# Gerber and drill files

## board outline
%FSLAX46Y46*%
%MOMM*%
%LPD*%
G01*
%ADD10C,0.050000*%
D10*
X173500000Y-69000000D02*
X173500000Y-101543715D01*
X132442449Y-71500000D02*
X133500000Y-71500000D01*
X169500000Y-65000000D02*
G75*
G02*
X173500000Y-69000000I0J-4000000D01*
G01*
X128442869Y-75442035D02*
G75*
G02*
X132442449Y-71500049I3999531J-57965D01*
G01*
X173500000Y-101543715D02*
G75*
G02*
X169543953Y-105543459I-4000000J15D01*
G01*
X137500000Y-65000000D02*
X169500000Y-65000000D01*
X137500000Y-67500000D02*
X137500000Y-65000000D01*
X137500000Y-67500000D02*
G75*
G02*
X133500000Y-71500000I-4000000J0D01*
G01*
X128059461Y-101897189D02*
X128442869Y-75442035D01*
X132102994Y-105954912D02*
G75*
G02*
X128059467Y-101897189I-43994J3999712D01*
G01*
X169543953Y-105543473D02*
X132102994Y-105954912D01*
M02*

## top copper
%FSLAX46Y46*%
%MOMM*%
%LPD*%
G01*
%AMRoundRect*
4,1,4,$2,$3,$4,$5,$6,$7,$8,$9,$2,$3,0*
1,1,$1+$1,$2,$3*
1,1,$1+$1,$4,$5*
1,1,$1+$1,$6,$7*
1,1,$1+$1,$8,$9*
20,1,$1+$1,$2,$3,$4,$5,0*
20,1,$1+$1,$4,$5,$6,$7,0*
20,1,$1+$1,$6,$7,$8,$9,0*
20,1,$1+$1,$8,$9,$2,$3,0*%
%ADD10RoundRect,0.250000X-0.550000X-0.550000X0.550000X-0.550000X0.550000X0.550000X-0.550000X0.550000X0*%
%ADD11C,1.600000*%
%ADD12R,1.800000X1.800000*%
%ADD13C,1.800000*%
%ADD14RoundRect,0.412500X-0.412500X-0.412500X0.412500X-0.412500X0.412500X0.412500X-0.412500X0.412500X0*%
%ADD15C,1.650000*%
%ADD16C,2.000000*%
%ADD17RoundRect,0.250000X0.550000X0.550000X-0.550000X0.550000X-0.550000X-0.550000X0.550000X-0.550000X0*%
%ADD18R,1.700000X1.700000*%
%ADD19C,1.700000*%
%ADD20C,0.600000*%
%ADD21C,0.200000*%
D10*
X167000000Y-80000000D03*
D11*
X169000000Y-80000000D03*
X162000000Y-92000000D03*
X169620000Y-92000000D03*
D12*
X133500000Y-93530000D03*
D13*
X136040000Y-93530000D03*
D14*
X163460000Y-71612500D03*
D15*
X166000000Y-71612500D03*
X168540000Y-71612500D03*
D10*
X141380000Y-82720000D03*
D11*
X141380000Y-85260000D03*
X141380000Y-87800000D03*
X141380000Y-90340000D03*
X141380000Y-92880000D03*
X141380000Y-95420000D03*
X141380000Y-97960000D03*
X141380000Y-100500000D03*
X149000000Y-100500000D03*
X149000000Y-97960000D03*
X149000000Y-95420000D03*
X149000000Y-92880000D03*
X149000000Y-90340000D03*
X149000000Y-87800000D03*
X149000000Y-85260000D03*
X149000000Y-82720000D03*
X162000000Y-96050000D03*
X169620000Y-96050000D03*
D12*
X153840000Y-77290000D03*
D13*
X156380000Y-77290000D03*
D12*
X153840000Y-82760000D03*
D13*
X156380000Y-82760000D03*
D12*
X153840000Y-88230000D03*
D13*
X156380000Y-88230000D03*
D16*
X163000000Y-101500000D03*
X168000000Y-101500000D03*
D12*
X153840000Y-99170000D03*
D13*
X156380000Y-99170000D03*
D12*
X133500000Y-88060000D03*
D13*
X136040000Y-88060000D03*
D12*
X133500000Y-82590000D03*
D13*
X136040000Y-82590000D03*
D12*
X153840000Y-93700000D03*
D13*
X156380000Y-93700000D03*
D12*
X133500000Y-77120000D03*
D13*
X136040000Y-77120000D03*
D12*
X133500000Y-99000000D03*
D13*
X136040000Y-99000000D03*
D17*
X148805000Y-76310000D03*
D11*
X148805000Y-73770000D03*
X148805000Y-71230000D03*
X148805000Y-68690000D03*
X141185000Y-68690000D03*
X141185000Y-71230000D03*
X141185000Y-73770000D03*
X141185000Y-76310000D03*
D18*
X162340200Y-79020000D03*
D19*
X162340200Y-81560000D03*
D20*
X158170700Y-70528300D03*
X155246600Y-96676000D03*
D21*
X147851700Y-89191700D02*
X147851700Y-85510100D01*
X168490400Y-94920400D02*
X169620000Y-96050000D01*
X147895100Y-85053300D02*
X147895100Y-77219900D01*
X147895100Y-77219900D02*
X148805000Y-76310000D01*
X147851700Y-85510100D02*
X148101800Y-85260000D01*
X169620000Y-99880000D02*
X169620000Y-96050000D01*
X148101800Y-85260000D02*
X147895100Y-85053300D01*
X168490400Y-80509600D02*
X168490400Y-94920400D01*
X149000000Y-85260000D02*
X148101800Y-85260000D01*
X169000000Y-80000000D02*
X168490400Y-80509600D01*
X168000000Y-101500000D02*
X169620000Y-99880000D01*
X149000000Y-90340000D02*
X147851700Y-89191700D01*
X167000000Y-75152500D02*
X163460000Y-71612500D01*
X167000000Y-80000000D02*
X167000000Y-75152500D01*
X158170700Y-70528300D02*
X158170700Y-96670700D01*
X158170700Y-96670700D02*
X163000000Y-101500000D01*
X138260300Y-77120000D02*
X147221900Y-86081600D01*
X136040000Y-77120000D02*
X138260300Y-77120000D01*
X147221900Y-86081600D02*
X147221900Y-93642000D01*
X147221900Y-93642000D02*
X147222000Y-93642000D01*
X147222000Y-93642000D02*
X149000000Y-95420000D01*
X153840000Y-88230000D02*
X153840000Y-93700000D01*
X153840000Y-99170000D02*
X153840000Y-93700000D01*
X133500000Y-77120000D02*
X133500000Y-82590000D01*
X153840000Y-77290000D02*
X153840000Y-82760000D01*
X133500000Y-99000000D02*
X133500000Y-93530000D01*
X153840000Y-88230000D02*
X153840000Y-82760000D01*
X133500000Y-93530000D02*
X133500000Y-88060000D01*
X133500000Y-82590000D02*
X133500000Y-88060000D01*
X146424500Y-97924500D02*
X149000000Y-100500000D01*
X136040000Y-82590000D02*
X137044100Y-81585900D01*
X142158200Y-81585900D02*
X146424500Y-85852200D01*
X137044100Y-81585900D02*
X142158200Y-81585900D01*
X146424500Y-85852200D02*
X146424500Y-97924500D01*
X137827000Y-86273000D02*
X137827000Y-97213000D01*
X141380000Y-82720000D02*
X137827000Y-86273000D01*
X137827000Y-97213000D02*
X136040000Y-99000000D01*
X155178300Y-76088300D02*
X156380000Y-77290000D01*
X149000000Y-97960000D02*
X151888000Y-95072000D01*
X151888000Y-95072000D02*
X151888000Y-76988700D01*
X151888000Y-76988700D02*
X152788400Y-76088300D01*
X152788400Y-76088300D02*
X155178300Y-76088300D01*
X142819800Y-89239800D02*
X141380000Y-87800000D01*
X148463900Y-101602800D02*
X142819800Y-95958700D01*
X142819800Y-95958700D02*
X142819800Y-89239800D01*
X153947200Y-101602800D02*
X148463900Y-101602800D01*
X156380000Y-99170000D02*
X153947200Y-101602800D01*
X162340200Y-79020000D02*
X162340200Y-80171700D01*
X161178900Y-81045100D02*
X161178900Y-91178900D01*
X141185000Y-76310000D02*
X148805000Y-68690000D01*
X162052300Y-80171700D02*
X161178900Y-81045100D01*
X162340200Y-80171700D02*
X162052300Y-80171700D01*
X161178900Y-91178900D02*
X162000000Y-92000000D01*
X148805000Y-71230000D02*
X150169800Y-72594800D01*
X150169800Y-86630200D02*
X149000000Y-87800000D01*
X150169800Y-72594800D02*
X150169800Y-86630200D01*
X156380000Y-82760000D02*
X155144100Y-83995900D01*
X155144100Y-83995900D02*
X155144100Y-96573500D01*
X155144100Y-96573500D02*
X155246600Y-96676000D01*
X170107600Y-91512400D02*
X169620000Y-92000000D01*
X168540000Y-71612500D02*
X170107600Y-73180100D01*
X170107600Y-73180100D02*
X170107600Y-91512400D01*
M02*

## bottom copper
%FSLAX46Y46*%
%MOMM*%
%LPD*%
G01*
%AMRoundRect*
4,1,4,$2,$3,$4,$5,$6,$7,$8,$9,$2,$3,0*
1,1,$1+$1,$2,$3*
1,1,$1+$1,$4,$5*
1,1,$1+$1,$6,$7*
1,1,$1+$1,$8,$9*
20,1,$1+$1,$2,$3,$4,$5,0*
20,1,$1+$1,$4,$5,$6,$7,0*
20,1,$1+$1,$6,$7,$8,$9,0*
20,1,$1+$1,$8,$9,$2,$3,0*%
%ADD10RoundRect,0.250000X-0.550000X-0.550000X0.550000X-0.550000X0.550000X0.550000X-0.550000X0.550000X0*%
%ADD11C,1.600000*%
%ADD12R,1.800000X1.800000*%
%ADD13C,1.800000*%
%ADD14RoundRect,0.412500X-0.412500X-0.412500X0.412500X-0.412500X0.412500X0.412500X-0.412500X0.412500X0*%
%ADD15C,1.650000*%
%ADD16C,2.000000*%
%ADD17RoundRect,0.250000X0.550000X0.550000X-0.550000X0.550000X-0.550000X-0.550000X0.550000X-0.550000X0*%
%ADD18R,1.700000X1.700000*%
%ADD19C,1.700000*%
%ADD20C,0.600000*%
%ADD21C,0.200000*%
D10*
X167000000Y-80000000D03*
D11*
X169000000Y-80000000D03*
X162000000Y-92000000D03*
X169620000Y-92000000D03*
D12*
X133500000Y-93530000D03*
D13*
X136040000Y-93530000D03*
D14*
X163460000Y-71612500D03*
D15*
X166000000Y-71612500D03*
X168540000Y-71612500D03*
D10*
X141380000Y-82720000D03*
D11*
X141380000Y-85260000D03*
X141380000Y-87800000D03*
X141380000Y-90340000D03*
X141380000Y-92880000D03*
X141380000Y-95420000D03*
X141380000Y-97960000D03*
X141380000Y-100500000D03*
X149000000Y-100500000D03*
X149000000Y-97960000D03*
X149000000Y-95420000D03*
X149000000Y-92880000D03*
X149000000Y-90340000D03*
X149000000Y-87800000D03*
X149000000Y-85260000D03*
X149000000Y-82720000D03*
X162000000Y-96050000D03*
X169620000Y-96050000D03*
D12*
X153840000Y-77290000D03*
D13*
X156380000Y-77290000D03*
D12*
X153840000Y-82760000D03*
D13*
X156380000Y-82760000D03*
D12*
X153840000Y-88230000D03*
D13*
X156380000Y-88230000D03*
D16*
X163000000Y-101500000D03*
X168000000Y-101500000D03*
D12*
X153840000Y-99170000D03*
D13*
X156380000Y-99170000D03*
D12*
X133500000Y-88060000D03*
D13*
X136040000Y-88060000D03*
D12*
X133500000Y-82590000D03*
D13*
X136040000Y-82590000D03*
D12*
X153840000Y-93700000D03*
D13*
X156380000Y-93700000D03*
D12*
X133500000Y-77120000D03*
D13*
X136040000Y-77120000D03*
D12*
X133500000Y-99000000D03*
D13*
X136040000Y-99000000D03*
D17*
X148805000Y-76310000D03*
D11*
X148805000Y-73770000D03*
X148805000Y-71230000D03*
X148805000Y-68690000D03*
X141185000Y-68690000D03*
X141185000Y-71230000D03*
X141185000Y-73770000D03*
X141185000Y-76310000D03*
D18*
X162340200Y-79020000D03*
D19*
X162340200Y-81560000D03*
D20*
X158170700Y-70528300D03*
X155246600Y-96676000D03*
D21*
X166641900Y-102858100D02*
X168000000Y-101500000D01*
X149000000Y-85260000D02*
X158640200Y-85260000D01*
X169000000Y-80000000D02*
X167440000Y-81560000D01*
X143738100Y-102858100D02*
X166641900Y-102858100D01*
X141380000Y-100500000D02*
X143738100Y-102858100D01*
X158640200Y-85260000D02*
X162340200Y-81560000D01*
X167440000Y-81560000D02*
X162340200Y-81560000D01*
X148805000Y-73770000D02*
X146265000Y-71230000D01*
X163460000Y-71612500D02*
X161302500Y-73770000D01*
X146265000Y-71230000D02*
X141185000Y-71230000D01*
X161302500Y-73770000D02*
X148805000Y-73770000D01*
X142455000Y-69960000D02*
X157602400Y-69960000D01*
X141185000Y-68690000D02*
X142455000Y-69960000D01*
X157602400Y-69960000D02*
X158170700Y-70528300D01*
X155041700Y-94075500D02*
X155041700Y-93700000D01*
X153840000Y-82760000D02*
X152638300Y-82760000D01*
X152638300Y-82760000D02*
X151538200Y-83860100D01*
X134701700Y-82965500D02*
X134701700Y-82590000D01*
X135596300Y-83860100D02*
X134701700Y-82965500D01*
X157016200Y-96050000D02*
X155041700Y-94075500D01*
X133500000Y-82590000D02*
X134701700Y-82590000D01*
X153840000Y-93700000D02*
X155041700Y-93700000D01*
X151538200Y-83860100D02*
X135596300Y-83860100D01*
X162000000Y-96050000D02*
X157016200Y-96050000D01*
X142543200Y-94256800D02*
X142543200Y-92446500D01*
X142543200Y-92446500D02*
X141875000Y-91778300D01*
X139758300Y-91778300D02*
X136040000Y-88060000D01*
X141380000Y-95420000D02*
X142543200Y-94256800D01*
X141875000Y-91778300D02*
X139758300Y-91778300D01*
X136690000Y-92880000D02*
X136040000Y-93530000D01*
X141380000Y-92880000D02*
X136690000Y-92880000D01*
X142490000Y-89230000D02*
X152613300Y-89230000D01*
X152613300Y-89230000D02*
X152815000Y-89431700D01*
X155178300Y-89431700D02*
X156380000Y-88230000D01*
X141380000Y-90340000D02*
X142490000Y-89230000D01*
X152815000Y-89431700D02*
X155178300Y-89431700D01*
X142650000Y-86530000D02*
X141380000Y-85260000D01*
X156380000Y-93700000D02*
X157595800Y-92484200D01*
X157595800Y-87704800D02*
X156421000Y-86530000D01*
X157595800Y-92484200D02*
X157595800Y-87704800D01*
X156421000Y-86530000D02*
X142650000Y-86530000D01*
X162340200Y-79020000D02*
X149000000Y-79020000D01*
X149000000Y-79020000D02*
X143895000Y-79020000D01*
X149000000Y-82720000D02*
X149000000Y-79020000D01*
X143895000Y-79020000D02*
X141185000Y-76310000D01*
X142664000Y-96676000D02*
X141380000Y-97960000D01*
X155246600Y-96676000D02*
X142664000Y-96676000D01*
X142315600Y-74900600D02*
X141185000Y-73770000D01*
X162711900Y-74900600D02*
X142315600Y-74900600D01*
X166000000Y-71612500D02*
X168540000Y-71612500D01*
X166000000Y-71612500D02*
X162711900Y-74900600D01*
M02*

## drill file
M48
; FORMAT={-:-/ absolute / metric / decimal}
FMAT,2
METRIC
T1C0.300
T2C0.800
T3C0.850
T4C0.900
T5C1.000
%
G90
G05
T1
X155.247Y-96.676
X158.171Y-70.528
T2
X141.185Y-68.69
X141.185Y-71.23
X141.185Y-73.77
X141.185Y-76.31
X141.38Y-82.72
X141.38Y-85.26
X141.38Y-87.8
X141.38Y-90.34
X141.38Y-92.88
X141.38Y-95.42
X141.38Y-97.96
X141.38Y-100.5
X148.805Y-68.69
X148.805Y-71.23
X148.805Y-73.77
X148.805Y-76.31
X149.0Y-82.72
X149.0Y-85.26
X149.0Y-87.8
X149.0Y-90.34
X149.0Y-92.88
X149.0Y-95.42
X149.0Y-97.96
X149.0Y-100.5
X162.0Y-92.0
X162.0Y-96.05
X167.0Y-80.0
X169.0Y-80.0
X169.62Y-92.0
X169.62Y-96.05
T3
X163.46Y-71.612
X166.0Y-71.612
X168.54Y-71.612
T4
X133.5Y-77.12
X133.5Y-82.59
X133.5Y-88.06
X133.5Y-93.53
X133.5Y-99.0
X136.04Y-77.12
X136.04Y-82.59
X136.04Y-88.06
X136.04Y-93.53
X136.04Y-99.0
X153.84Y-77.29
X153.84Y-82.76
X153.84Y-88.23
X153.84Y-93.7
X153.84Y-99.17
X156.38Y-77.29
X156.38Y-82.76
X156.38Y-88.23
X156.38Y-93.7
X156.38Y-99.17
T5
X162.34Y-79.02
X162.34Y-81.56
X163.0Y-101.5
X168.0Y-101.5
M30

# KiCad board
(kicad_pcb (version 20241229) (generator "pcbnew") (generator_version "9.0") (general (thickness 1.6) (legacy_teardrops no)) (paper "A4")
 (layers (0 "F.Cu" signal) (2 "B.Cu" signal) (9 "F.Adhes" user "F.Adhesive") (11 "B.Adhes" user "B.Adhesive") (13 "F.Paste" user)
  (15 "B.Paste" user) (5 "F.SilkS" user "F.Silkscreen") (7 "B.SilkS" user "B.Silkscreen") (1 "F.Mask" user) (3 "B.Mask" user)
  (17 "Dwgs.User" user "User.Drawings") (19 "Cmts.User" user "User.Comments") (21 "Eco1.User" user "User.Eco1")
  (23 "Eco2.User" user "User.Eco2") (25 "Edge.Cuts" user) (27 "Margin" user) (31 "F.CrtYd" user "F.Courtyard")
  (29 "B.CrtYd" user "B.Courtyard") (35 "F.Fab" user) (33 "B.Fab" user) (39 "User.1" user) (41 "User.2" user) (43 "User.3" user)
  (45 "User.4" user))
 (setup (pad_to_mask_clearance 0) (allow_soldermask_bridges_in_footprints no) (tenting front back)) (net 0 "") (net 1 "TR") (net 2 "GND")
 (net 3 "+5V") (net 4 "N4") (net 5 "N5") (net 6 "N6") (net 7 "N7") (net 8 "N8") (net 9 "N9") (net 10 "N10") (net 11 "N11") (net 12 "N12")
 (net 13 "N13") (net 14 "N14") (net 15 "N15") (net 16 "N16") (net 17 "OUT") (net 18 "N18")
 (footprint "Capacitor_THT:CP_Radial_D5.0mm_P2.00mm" (layer "F.Cu") (at 167 80)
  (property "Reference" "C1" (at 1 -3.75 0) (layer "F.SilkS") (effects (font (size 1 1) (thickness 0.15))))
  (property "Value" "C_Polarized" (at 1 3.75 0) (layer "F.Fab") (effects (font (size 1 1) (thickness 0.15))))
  (pad "1" thru_hole roundrect (at 0 0) (size 1.6 1.6) (drill 0.8) (layers "*.Cu" "*.Mask") (remove_unused_layers no)
   (roundrect_rratio 0.15625) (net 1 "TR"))
  (pad "2" thru_hole circle (at 2 0) (size 1.6 1.6) (drill 0.8) (layers "*.Cu" "*.Mask") (remove_unused_layers no) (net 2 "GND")))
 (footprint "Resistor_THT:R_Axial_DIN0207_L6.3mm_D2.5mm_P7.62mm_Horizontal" (layer "F.Cu") (at 162 92)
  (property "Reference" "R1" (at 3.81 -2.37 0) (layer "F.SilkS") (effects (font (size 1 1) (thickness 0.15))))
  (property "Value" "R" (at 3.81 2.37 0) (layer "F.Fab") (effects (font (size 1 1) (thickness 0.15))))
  (pad "1" thru_hole circle (at 0 0) (size 1.6 1.6) (drill 0.8) (layers "*.Cu" "*.Mask") (remove_unused_layers no) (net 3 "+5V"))
  (pad "2" thru_hole circle (at 7.62 0) (size 1.6 1.6) (drill 0.8) (layers "*.Cu" "*.Mask") (remove_unused_layers no) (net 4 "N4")))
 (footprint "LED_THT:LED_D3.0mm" (layer "F.Cu") (at 133.5 93.53)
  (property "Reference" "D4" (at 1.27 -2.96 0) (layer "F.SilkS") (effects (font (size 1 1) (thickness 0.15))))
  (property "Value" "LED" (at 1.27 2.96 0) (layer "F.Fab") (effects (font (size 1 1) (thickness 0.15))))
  (pad "1" thru_hole rect (at 0 0) (size 1.8 1.8) (drill 0.9) (layers "*.Cu" "*.Mask") (remove_unused_layers no) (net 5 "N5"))
  (pad "2" thru_hole circle (at 2.54 0) (size 1.8 1.8) (drill 0.9) (layers "*.Cu" "*.Mask") (remove_unused_layers no) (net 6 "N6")))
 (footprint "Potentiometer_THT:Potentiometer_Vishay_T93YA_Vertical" (layer "F.Cu") (at 163.46 71.6125)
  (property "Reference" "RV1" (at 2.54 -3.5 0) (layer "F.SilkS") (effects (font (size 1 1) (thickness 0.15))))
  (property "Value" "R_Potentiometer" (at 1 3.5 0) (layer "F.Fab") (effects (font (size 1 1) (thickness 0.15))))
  (pad "1" thru_hole roundrect (at 0 0) (size 1.65 1.65) (drill 0.85) (layers "*.Cu" "*.Mask") (remove_unused_layers no)
   (roundrect_rratio 0.25) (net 1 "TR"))
  (pad "2" thru_hole circle (at 2.54 0) (size 1.65 1.65) (drill 0.85) (layers "*.Cu" "*.Mask") (remove_unused_layers no) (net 4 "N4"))
  (pad "3" thru_hole circle (at 5.08 0) (size 1.65 1.65) (drill 0.85) (layers "*.Cu" "*.Mask") (remove_unused_layers no) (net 4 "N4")))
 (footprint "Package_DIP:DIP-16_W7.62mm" (layer "F.Cu") (at 141.38 82.72)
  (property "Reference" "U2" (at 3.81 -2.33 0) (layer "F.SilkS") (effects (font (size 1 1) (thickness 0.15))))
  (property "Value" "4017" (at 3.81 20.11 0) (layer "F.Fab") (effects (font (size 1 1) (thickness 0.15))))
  (pad "1" thru_hole roundrect (at 0 0) (size 1.6 1.6) (drill 0.8) (layers "*.Cu" "*.Mask") (remove_unused_layers no)
   (roundrect_rratio 0.15625) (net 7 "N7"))
  (pad "2" thru_hole circle (at 0 2.54) (size 1.6 1.6) (drill 0.8) (layers "*.Cu" "*.Mask") (remove_unused_layers no) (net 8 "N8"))
  (pad "3" thru_hole circle (at 0 5.08) (size 1.6 1.6) (drill 0.8) (layers "*.Cu" "*.Mask") (remove_unused_layers no) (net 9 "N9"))
  (pad "4" thru_hole circle (at 0 7.62) (size 1.6 1.6) (drill 0.8) (layers "*.Cu" "*.Mask") (remove_unused_layers no) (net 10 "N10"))
  (pad "5" thru_hole circle (at 0 10.16) (size 1.6 1.6) (drill 0.8) (layers "*.Cu" "*.Mask") (remove_unused_layers no) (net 6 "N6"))
  (pad "6" thru_hole circle (at 0 12.7) (size 1.6 1.6) (drill 0.8) (layers "*.Cu" "*.Mask") (remove_unused_layers no) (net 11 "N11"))
  (pad "7" thru_hole circle (at 0 15.24) (size 1.6 1.6) (drill 0.8) (layers "*.Cu" "*.Mask") (remove_unused_layers no) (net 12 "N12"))
  (pad "8" thru_hole circle (at 0 17.78) (size 1.6 1.6) (drill 0.8) (layers "*.Cu" "*.Mask") (remove_unused_layers no) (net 2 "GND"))
  (pad "9" thru_hole circle (at 7.62 17.78) (size 1.6 1.6) (drill 0.8) (layers "*.Cu" "*.Mask") (remove_unused_layers no) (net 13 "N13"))
  (pad "10" thru_hole circle (at 7.62 15.24) (size 1.6 1.6) (drill 0.8) (layers "*.Cu" "*.Mask") (remove_unused_layers no) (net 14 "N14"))
  (pad "11" thru_hole circle (at 7.62 12.7) (size 1.6 1.6) (drill 0.8) (layers "*.Cu" "*.Mask") (remove_unused_layers no) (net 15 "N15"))
  (pad "12" thru_hole circle (at 7.62 10.16) (size 1.6 1.6) (drill 0.8) (layers "*.Cu" "*.Mask") (remove_unused_layers no) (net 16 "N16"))
  (pad "13" thru_hole circle (at 7.62 7.62) (size 1.6 1.6) (drill 0.8) (layers "*.Cu" "*.Mask") (remove_unused_layers no) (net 2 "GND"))
  (pad "14" thru_hole circle (at 7.62 5.08) (size 1.6 1.6) (drill 0.8) (layers "*.Cu" "*.Mask") (remove_unused_layers no) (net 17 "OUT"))
  (pad "15" thru_hole circle (at 7.62 2.54) (size 1.6 1.6) (drill 0.8) (layers "*.Cu" "*.Mask") (remove_unused_layers no) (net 2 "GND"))
  (pad "16" thru_hole circle (at 7.62 0) (size 1.6 1.6) (drill 0.8) (layers "*.Cu" "*.Mask") (remove_unused_layers no) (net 3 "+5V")))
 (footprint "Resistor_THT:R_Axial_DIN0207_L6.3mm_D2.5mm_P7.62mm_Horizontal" (layer "F.Cu") (at 162 96.05)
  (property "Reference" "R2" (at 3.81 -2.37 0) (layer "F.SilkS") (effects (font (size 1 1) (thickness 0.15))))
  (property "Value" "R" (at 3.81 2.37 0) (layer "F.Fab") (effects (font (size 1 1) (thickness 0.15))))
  (pad "1" thru_hole circle (at 0 0) (size 1.6 1.6) (drill 0.8) (layers "*.Cu" "*.Mask") (remove_unused_layers no) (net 5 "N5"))
  (pad "2" thru_hole circle (at 7.62 0) (size 1.6 1.6) (drill 0.8) (layers "*.Cu" "*.Mask") (remove_unused_layers no) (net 2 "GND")))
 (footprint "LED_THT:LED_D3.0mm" (layer "F.Cu") (at 153.84 77.29)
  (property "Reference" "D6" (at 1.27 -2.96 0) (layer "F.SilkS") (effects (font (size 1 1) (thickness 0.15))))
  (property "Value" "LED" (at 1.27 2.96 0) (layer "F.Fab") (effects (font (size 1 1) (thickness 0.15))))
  (pad "1" thru_hole rect (at 0 0) (size 1.8 1.8) (drill 0.9) (layers "*.Cu" "*.Mask") (remove_unused_layers no) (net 5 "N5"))
  (pad "2" thru_hole circle (at 2.54 0) (size 1.8 1.8) (drill 0.9) (layers "*.Cu" "*.Mask") (remove_unused_layers no) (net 14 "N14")))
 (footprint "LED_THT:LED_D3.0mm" (layer "F.Cu") (at 153.84 82.76)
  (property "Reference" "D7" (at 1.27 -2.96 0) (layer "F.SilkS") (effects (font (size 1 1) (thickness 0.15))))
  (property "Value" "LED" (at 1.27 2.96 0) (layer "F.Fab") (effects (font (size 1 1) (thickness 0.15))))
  (pad "1" thru_hole rect (at 0 0) (size 1.8 1.8) (drill 0.9) (layers "*.Cu" "*.Mask") (remove_unused_layers no) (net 5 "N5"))
  (pad "2" thru_hole circle (at 2.54 0) (size 1.8 1.8) (drill 0.9) (layers "*.Cu" "*.Mask") (remove_unused_layers no) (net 12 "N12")))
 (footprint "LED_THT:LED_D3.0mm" (layer "F.Cu") (at 153.84 88.23)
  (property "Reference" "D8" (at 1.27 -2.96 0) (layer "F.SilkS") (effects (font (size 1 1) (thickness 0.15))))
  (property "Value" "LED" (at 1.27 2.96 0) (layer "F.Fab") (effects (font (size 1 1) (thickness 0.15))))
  (pad "1" thru_hole rect (at 0 0) (size 1.8 1.8) (drill 0.9) (layers "*.Cu" "*.Mask") (remove_unused_layers no) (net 5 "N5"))
  (pad "2" thru_hole circle (at 2.54 0) (size 1.8 1.8) (drill 0.9) (layers "*.Cu" "*.Mask") (remove_unused_layers no) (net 10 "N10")))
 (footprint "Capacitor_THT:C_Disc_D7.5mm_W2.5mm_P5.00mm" (layer "F.Cu") (at 163 101.5)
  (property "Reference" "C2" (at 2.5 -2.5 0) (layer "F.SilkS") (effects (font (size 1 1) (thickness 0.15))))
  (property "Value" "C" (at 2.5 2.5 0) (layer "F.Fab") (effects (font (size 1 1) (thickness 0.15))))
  (pad "1" thru_hole circle (at 0 0) (size 2 2) (drill 1) (layers "*.Cu" "*.Mask") (remove_unused_layers no) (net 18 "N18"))
  (pad "2" thru_hole circle (at 5 0) (size 2 2) (drill 1) (layers "*.Cu" "*.Mask") (remove_unused_layers no) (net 2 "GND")))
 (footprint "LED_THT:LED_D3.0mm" (layer "F.Cu") (at 153.84 99.17)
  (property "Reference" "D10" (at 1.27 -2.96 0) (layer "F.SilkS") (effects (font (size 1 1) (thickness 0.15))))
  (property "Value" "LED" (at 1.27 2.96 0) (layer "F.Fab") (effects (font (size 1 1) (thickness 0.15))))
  (pad "1" thru_hole rect (at 0 0) (size 1.8 1.8) (drill 0.9) (layers "*.Cu" "*.Mask") (remove_unused_layers no) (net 5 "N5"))
  (pad "2" thru_hole circle (at 2.54 0) (size 1.8 1.8) (drill 0.9) (layers "*.Cu" "*.Mask") (remove_unused_layers no) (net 9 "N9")))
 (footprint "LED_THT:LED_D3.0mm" (layer "F.Cu") (at 133.5 88.06)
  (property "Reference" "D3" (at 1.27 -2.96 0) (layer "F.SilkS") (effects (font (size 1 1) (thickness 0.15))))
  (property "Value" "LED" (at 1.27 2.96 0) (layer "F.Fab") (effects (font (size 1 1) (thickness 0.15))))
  (pad "1" thru_hole rect (at 0 0) (size 1.8 1.8) (drill 0.9) (layers "*.Cu" "*.Mask") (remove_unused_layers no) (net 5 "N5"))
  (pad "2" thru_hole circle (at 2.54 0) (size 1.8 1.8) (drill 0.9) (layers "*.Cu" "*.Mask") (remove_unused_layers no) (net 11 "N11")))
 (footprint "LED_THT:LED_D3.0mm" (layer "F.Cu") (at 133.5 82.59)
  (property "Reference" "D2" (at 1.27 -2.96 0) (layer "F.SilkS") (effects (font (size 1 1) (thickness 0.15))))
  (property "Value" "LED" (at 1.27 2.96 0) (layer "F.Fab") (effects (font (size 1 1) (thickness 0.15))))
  (pad "1" thru_hole rect (at 0 0) (size 1.8 1.8) (drill 0.9) (layers "*.Cu" "*.Mask") (remove_unused_layers no) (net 5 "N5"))
  (pad "2" thru_hole circle (at 2.54 0) (size 1.8 1.8) (drill 0.9) (layers "*.Cu" "*.Mask") (remove_unused_layers no) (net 13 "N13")))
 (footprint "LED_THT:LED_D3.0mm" (layer "F.Cu") (at 153.84 93.7)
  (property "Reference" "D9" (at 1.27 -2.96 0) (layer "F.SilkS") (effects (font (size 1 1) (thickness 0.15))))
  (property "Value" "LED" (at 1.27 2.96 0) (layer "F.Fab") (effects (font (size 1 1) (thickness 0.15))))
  (pad "1" thru_hole rect (at 0 0) (size 1.8 1.8) (drill 0.9) (layers "*.Cu" "*.Mask") (remove_unused_layers no) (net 5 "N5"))
  (pad "2" thru_hole circle (at 2.54 0) (size 1.8 1.8) (drill 0.9) (layers "*.Cu" "*.Mask") (remove_unused_layers no) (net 8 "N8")))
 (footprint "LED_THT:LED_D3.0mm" (layer "F.Cu") (at 133.5 77.12)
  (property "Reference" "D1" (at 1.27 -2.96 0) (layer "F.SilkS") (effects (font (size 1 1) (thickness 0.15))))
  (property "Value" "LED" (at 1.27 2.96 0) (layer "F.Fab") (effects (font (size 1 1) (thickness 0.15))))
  (pad "1" thru_hole rect (at 0 0) (size 1.8 1.8) (drill 0.9) (layers "*.Cu" "*.Mask") (remove_unused_layers no) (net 5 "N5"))
  (pad "2" thru_hole circle (at 2.54 0) (size 1.8 1.8) (drill 0.9) (layers "*.Cu" "*.Mask") (remove_unused_layers no) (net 15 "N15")))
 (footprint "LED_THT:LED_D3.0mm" (layer "F.Cu") (at 133.5 99)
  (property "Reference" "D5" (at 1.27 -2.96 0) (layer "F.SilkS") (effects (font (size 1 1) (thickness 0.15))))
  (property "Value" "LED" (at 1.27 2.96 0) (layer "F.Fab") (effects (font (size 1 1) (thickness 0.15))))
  (pad "1" thru_hole rect (at 0 0) (size 1.8 1.8) (drill 0.9) (layers "*.Cu" "*.Mask") (remove_unused_layers no) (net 5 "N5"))
  (pad "2" thru_hole circle (at 2.54 0) (size 1.8 1.8) (drill 0.9) (layers "*.Cu" "*.Mask") (remove_unused_layers no) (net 7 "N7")))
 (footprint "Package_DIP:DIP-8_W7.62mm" (layer "F.Cu") (at 148.805 76.31 180)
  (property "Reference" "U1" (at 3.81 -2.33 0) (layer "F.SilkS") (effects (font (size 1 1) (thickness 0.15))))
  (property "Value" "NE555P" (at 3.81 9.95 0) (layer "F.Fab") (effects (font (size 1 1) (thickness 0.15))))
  (pad "1" thru_hole roundrect (at 0 0 180) (size 1.6 1.6) (drill 0.8) (layers "*.Cu" "*.Mask") (remove_unused_layers no)
   (roundrect_rratio 0.15625) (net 2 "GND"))
  (pad "2" thru_hole circle (at 0 2.54 180) (size 1.6 1.6) (drill 0.8) (layers "*.Cu" "*.Mask") (remove_unused_layers no) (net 1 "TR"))
  (pad "3" thru_hole circle (at 0 5.08 180) (size 1.6 1.6) (drill 0.8) (layers "*.Cu" "*.Mask") (remove_unused_layers no) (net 17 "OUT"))
  (pad "4" thru_hole circle (at 0 7.62 180) (size 1.6 1.6) (drill 0.8) (layers "*.Cu" "*.Mask") (remove_unused_layers no) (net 3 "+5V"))
  (pad "5" thru_hole circle (at 7.62 7.62 180) (size 1.6 1.6) (drill 0.8) (layers "*.Cu" "*.Mask") (remove_unused_layers no) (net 18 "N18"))
  (pad "6" thru_hole circle (at 7.62 5.08 180) (size 1.6 1.6) (drill 0.8) (layers "*.Cu" "*.Mask") (remove_unused_layers no) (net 1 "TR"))
  (pad "7" thru_hole circle (at 7.62 2.54 180) (size 1.6 1.6) (drill 0.8) (layers "*.Cu" "*.Mask") (remove_unused_layers no) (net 4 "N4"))
  (pad "8" thru_hole circle (at 7.62 0 180) (size 1.6 1.6) (drill 0.8) (layers "*.Cu" "*.Mask") (remove_unused_layers no) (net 3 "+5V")))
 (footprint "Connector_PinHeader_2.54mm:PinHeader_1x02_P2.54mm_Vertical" (layer "F.Cu") (at 162.3402 79.02)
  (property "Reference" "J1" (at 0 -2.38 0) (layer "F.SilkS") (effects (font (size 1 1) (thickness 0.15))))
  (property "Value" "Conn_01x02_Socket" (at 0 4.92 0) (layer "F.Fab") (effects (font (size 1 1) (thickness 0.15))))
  (pad "1" thru_hole rect (at 0 0) (size 1.7 1.7) (drill 1) (layers "*.Cu" "*.Mask") (remove_unused_layers no) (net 3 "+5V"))
  (pad "2" thru_hole circle (at 0 2.54) (size 1.7 1.7) (drill 1) (layers "*.Cu" "*.Mask") (remove_unused_layers no) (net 2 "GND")))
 (gr_line (start 173.5 69) (end 173.5 101.543715) (stroke (width 0.05) (type default)) (layer "Edge.Cuts"))
 (gr_line (start 132.442449 71.5) (end 133.5 71.5) (stroke (width 0.05) (type default)) (layer "Edge.Cuts"))
 (gr_arc (start 169.5 65) (mid 172.328427 66.171573) (end 173.5 69) (stroke (width 0.05) (type default)) (layer "Edge.Cuts"))
 (gr_arc (start 128.442869 75.442035) (mid 129.63459 72.651153) (end 132.442449 71.5) (stroke (width 0.05) (type default))
  (layer "Edge.Cuts"))
 (gr_arc (start 173.5 101.543715) (mid 172.343924 104.356559) (end 169.543953 105.543473) (stroke (width 0.05) (type default))
  (layer "Edge.Cuts"))
 (gr_line (start 137.5 65) (end 169.5 65) (stroke (width 0.05) (type default)) (layer "Edge.Cuts"))
 (gr_line (start 137.5 67.5) (end 137.5 65) (stroke (width 0.05) (type default)) (layer "Edge.Cuts"))
 (gr_arc (start 137.5 67.5) (mid 136.328427 70.328427) (end 133.5 71.5) (stroke (width 0.05) (type default)) (layer "Edge.Cuts"))
 (gr_line (start 128.059461 101.897189) (end 128.442869 75.442035) (stroke (width 0.05) (type default)) (layer "Edge.Cuts"))
 (gr_arc (start 132.102994 105.954912) (mid 129.225662 104.778623) (end 128.059461 101.897189) (stroke (width 0.05) (type default))
  (layer "Edge.Cuts"))
 (gr_line (start 169.543953 105.543473) (end 132.102994 105.954912) (stroke (width 0.05) (type default)) (layer "Edge.Cuts"))
 (segment (start 147.8517 89.1917) (end 147.8517 85.5101) (width 0.2) (layer "F.Cu") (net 2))
 (segment (start 168.4904 94.9204) (end 169.62 96.05) (width 0.2) (layer "F.Cu") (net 2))
 (segment (start 147.8951 85.0533) (end 147.8951 77.2199) (width 0.2) (layer "F.Cu") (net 2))
 (segment (start 147.8951 77.2199) (end 148.805 76.31) (width 0.2) (layer "F.Cu") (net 2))
 (segment (start 147.8517 85.5101) (end 148.1018 85.26) (width 0.2) (layer "F.Cu") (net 2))
 (segment (start 169.62 99.88) (end 169.62 96.05) (width 0.2) (layer "F.Cu") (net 2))
 (segment (start 148.1018 85.26) (end 147.8951 85.0533) (width 0.2) (layer "F.Cu") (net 2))
 (segment (start 168.4904 80.5096) (end 168.4904 94.9204) (width 0.2) (layer "F.Cu") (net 2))
 (segment (start 149 85.26) (end 148.1018 85.26) (width 0.2) (layer "F.Cu") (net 2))
 (segment (start 169 80) (end 168.4904 80.5096) (width 0.2) (layer "F.Cu") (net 2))
 (segment (start 168 101.5) (end 169.62 99.88) (width 0.2) (layer "F.Cu") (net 2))
 (segment (start 149 90.34) (end 147.8517 89.1917) (width 0.2) (layer "F.Cu") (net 2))
 (segment (start 166.6419 102.8581) (end 168 101.5) (width 0.2) (layer "B.Cu") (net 2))
 (segment (start 149 85.26) (end 158.6402 85.26) (width 0.2) (layer "B.Cu") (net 2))
 (segment (start 169 80) (end 167.44 81.56) (width 0.2) (layer "B.Cu") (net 2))
 (segment (start 143.7381 102.8581) (end 166.6419 102.8581) (width 0.2) (layer "B.Cu") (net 2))
 (segment (start 141.38 100.5) (end 143.7381 102.8581) (width 0.2) (layer "B.Cu") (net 2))
 (segment (start 158.6402 85.26) (end 162.3402 81.56) (width 0.2) (layer "B.Cu") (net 2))
 (segment (start 167.44 81.56) (end 162.3402 81.56) (width 0.2) (layer "B.Cu") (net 2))
 (segment (start 167 75.1525) (end 163.46 71.6125) (width 0.2) (layer "F.Cu") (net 1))
 (segment (start 167 80) (end 167 75.1525) (width 0.2) (layer "F.Cu") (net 1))
 (segment (start 148.805 73.77) (end 146.265 71.23) (width 0.2) (layer "B.Cu") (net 1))
 (segment (start 163.46 71.6125) (end 161.3025 73.77) (width 0.2) (layer "B.Cu") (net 1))
 (segment (start 146.265 71.23) (end 141.185 71.23) (width 0.2) (layer "B.Cu") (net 1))
 (segment (start 161.3025 73.77) (end 148.805 73.77) (width 0.2) (layer "B.Cu") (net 1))
 (segment (start 158.1707 70.5283) (end 158.1707 96.6707) (width 0.2) (layer "F.Cu") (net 18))
 (segment (start 158.1707 96.6707) (end 163 101.5) (width 0.2) (layer "F.Cu") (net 18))
 (via (at 158.1707 70.5283) (size 0.6) (drill 0.3) (layers "F.Cu" "B.Cu") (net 18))
 (segment (start 142.455 69.96) (end 157.6024 69.96) (width 0.2) (layer "B.Cu") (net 18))
 (segment (start 141.185 68.69) (end 142.455 69.96) (width 0.2) (layer "B.Cu") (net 18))
 (segment (start 157.6024 69.96) (end 158.1707 70.5283) (width 0.2) (layer "B.Cu") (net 18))
 (segment (start 138.2603 77.12) (end 147.2219 86.0816) (width 0.2) (layer "F.Cu") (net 15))
 (segment (start 136.04 77.12) (end 138.2603 77.12) (width 0.2) (layer "F.Cu") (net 15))
 (segment (start 147.2219 86.0816) (end 147.2219 93.642) (width 0.2) (layer "F.Cu") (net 15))
 (segment (start 147.2219 93.642) (end 147.222 93.642) (width 0.2) (layer "F.Cu") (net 15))
 (segment (start 147.222 93.642) (end 149 95.42) (width 0.2) (layer "F.Cu") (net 15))
 (segment (start 153.84 88.23) (end 153.84 93.7) (width 0.2) (layer "F.Cu") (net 5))
 (segment (start 153.84 99.17) (end 153.84 93.7) (width 0.2) (layer "F.Cu") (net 5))
 (segment (start 133.5 77.12) (end 133.5 82.59) (width 0.2) (layer "F.Cu") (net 5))
 (segment (start 153.84 77.29) (end 153.84 82.76) (width 0.2) (layer "F.Cu") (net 5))
 (segment (start 133.5 99) (end 133.5 93.53) (width 0.2) (layer "F.Cu") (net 5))
 (segment (start 153.84 88.23) (end 153.84 82.76) (width 0.2) (layer "F.Cu") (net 5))
 (segment (start 133.5 93.53) (end 133.5 88.06) (width 0.2) (layer "F.Cu") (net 5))
 (segment (start 133.5 82.59) (end 133.5 88.06) (width 0.2) (layer "F.Cu") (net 5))
 (segment (start 155.0417 94.0755) (end 155.0417 93.7) (width 0.2) (layer "B.Cu") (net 5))
 (segment (start 153.84 82.76) (end 152.6383 82.76) (width 0.2) (layer "B.Cu") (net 5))
 (segment (start 152.6383 82.76) (end 151.5382 83.8601) (width 0.2) (layer "B.Cu") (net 5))
 (segment (start 134.7017 82.9655) (end 134.7017 82.59) (width 0.2) (layer "B.Cu") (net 5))
 (segment (start 135.5963 83.8601) (end 134.7017 82.9655) (width 0.2) (layer "B.Cu") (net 5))
 (segment (start 157.0162 96.05) (end 155.0417 94.0755) (width 0.2) (layer "B.Cu") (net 5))
 (segment (start 133.5 82.59) (end 134.7017 82.59) (width 0.2) (layer "B.Cu") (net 5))
 (segment (start 153.84 93.7) (end 155.0417 93.7) (width 0.2) (layer "B.Cu") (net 5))
 (segment (start 151.5382 83.8601) (end 135.5963 83.8601) (width 0.2) (layer "B.Cu") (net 5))
 (segment (start 162 96.05) (end 157.0162 96.05) (width 0.2) (layer "B.Cu") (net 5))
 (segment (start 146.4245 97.9245) (end 149 100.5) (width 0.2) (layer "F.Cu") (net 13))
 (segment (start 136.04 82.59) (end 137.0441 81.5859) (width 0.2) (layer "F.Cu") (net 13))
 (segment (start 142.1582 81.5859) (end 146.4245 85.8522) (width 0.2) (layer "F.Cu") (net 13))
 (segment (start 137.0441 81.5859) (end 142.1582 81.5859) (width 0.2) (layer "F.Cu") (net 13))
 (segment (start 146.4245 85.8522) (end 146.4245 97.9245) (width 0.2) (layer "F.Cu") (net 13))
 (segment (start 142.5432 94.2568) (end 142.5432 92.4465) (width 0.2) (layer "B.Cu") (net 11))
 (segment (start 142.5432 92.4465) (end 141.875 91.7783) (width 0.2) (layer "B.Cu") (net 11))
 (segment (start 139.7583 91.7783) (end 136.04 88.06) (width 0.2) (layer "B.Cu") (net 11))
 (segment (start 141.38 95.42) (end 142.5432 94.2568) (width 0.2) (layer "B.Cu") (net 11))
 (segment (start 141.875 91.7783) (end 139.7583 91.7783) (width 0.2) (layer "B.Cu") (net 11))
 (segment (start 136.69 92.88) (end 136.04 93.53) (width 0.2) (layer "B.Cu") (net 6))
 (segment (start 141.38 92.88) (end 136.69 92.88) (width 0.2) (layer "B.Cu") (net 6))
 (segment (start 137.827 86.273) (end 137.827 97.213) (width 0.2) (layer "F.Cu") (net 7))
 (segment (start 141.38 82.72) (end 137.827 86.273) (width 0.2) (layer "F.Cu") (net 7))
 (segment (start 137.827 97.213) (end 136.04 99) (width 0.2) (layer "F.Cu") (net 7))
 (segment (start 155.1783 76.0883) (end 156.38 77.29) (width 0.2) (layer "F.Cu") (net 14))
 (segment (start 149 97.96) (end 151.888 95.072) (width 0.2) (layer "F.Cu") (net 14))
 (segment (start 151.888 95.072) (end 151.888 76.9887) (width 0.2) (layer "F.Cu") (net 14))
 (segment (start 151.888 76.9887) (end 152.7884 76.0883) (width 0.2) (layer "F.Cu") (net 14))
 (segment (start 152.7884 76.0883) (end 155.1783 76.0883) (width 0.2) (layer "F.Cu") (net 14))
 (segment (start 142.49 89.23) (end 152.6133 89.23) (width 0.2) (layer "B.Cu") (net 10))
 (segment (start 152.6133 89.23) (end 152.815 89.4317) (width 0.2) (layer "B.Cu") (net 10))
 (segment (start 155.1783 89.4317) (end 156.38 88.23) (width 0.2) (layer "B.Cu") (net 10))
 (segment (start 141.38 90.34) (end 142.49 89.23) (width 0.2) (layer "B.Cu") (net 10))
 (segment (start 152.815 89.4317) (end 155.1783 89.4317) (width 0.2) (layer "B.Cu") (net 10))
 (segment (start 142.65 86.53) (end 141.38 85.26) (width 0.2) (layer "B.Cu") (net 8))
 (segment (start 156.38 93.7) (end 157.5958 92.4842) (width 0.2) (layer "B.Cu") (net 8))
 (segment (start 157.5958 87.7048) (end 156.421 86.53) (width 0.2) (layer "B.Cu") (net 8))
 (segment (start 157.5958 92.4842) (end 157.5958 87.7048) (width 0.2) (layer "B.Cu") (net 8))
 (segment (start 156.421 86.53) (end 142.65 86.53) (width 0.2) (layer "B.Cu") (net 8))
 (segment (start 142.8198 89.2398) (end 141.38 87.8) (width 0.2) (layer "F.Cu") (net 9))
 (segment (start 148.4639 101.6028) (end 142.8198 95.9587) (width 0.2) (layer "F.Cu") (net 9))
 (segment (start 142.8198 95.9587) (end 142.8198 89.2398) (width 0.2) (layer "F.Cu") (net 9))
 (segment (start 153.9472 101.6028) (end 148.4639 101.6028) (width 0.2) (layer "F.Cu") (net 9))
 (segment (start 156.38 99.17) (end 153.9472 101.6028) (width 0.2) (layer "F.Cu") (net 9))
 (segment (start 162.3402 79.02) (end 162.3402 80.1717) (width 0.2) (layer "F.Cu") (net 3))
 (segment (start 161.1789 81.0451) (end 161.1789 91.1789) (width 0.2) (layer "F.Cu") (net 3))
 (segment (start 141.185 76.31) (end 148.805 68.69) (width 0.2) (layer "F.Cu") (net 3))
 (segment (start 162.0523 80.1717) (end 161.1789 81.0451) (width 0.2) (layer "F.Cu") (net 3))
 (segment (start 162.3402 80.1717) (end 162.0523 80.1717) (width 0.2) (layer "F.Cu") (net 3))
 (segment (start 161.1789 91.1789) (end 162 92) (width 0.2) (layer "F.Cu") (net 3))
 (segment (start 162.3402 79.02) (end 149 79.02) (width 0.2) (layer "B.Cu") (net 3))
 (segment (start 149 79.02) (end 143.895 79.02) (width 0.2) (layer "B.Cu") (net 3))
 (segment (start 149 82.72) (end 149 79.02) (width 0.2) (layer "B.Cu") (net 3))
 (segment (start 143.895 79.02) (end 141.185 76.31) (width 0.2) (layer "B.Cu") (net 3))
 (segment (start 148.805 71.23) (end 150.1698 72.5948) (width 0.2) (layer "F.Cu") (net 17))
 (segment (start 150.1698 86.6302) (end 149 87.8) (width 0.2) (layer "F.Cu") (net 17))
 (segment (start 150.1698 72.5948) (end 150.1698 86.6302) (width 0.2) (layer "F.Cu") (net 17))
 (segment (start 156.38 82.76) (end 155.1441 83.9959) (width 0.2) (layer "F.Cu") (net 12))
 (segment (start 155.1441 83.9959) (end 155.1441 96.5735) (width 0.2) (layer "F.Cu") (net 12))
 (segment (start 155.1441 96.5735) (end 155.2466 96.676) (width 0.2) (layer "F.Cu") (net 12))
 (via (at 155.2466 96.676) (size 0.6) (drill 0.3) (layers "F.Cu" "B.Cu") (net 12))
 (segment (start 142.664 96.676) (end 141.38 97.96) (width 0.2) (layer "B.Cu") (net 12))
 (segment (start 155.2466 96.676) (end 142.664 96.676) (width 0.2) (layer "B.Cu") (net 12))
 (segment (start 170.1076 91.5124) (end 169.62 92) (width 0.2) (layer "F.Cu") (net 4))
 (segment (start 168.54 71.6125) (end 170.1076 73.1801) (width 0.2) (layer "F.Cu") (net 4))
 (segment (start 170.1076 73.1801) (end 170.1076 91.5124) (width 0.2) (layer "F.Cu") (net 4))
 (segment (start 142.3156 74.9006) (end 141.185 73.77) (width 0.2) (layer "B.Cu") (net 4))
 (segment (start 162.7119 74.9006) (end 142.3156 74.9006) (width 0.2) (layer "B.Cu") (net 4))
 (segment (start 166 71.6125) (end 168.54 71.6125) (width 0.2) (layer "B.Cu") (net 4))
 (segment (start 166 71.6125) (end 162.7119 74.9006) (width 0.2) (layer "B.Cu") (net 4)))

